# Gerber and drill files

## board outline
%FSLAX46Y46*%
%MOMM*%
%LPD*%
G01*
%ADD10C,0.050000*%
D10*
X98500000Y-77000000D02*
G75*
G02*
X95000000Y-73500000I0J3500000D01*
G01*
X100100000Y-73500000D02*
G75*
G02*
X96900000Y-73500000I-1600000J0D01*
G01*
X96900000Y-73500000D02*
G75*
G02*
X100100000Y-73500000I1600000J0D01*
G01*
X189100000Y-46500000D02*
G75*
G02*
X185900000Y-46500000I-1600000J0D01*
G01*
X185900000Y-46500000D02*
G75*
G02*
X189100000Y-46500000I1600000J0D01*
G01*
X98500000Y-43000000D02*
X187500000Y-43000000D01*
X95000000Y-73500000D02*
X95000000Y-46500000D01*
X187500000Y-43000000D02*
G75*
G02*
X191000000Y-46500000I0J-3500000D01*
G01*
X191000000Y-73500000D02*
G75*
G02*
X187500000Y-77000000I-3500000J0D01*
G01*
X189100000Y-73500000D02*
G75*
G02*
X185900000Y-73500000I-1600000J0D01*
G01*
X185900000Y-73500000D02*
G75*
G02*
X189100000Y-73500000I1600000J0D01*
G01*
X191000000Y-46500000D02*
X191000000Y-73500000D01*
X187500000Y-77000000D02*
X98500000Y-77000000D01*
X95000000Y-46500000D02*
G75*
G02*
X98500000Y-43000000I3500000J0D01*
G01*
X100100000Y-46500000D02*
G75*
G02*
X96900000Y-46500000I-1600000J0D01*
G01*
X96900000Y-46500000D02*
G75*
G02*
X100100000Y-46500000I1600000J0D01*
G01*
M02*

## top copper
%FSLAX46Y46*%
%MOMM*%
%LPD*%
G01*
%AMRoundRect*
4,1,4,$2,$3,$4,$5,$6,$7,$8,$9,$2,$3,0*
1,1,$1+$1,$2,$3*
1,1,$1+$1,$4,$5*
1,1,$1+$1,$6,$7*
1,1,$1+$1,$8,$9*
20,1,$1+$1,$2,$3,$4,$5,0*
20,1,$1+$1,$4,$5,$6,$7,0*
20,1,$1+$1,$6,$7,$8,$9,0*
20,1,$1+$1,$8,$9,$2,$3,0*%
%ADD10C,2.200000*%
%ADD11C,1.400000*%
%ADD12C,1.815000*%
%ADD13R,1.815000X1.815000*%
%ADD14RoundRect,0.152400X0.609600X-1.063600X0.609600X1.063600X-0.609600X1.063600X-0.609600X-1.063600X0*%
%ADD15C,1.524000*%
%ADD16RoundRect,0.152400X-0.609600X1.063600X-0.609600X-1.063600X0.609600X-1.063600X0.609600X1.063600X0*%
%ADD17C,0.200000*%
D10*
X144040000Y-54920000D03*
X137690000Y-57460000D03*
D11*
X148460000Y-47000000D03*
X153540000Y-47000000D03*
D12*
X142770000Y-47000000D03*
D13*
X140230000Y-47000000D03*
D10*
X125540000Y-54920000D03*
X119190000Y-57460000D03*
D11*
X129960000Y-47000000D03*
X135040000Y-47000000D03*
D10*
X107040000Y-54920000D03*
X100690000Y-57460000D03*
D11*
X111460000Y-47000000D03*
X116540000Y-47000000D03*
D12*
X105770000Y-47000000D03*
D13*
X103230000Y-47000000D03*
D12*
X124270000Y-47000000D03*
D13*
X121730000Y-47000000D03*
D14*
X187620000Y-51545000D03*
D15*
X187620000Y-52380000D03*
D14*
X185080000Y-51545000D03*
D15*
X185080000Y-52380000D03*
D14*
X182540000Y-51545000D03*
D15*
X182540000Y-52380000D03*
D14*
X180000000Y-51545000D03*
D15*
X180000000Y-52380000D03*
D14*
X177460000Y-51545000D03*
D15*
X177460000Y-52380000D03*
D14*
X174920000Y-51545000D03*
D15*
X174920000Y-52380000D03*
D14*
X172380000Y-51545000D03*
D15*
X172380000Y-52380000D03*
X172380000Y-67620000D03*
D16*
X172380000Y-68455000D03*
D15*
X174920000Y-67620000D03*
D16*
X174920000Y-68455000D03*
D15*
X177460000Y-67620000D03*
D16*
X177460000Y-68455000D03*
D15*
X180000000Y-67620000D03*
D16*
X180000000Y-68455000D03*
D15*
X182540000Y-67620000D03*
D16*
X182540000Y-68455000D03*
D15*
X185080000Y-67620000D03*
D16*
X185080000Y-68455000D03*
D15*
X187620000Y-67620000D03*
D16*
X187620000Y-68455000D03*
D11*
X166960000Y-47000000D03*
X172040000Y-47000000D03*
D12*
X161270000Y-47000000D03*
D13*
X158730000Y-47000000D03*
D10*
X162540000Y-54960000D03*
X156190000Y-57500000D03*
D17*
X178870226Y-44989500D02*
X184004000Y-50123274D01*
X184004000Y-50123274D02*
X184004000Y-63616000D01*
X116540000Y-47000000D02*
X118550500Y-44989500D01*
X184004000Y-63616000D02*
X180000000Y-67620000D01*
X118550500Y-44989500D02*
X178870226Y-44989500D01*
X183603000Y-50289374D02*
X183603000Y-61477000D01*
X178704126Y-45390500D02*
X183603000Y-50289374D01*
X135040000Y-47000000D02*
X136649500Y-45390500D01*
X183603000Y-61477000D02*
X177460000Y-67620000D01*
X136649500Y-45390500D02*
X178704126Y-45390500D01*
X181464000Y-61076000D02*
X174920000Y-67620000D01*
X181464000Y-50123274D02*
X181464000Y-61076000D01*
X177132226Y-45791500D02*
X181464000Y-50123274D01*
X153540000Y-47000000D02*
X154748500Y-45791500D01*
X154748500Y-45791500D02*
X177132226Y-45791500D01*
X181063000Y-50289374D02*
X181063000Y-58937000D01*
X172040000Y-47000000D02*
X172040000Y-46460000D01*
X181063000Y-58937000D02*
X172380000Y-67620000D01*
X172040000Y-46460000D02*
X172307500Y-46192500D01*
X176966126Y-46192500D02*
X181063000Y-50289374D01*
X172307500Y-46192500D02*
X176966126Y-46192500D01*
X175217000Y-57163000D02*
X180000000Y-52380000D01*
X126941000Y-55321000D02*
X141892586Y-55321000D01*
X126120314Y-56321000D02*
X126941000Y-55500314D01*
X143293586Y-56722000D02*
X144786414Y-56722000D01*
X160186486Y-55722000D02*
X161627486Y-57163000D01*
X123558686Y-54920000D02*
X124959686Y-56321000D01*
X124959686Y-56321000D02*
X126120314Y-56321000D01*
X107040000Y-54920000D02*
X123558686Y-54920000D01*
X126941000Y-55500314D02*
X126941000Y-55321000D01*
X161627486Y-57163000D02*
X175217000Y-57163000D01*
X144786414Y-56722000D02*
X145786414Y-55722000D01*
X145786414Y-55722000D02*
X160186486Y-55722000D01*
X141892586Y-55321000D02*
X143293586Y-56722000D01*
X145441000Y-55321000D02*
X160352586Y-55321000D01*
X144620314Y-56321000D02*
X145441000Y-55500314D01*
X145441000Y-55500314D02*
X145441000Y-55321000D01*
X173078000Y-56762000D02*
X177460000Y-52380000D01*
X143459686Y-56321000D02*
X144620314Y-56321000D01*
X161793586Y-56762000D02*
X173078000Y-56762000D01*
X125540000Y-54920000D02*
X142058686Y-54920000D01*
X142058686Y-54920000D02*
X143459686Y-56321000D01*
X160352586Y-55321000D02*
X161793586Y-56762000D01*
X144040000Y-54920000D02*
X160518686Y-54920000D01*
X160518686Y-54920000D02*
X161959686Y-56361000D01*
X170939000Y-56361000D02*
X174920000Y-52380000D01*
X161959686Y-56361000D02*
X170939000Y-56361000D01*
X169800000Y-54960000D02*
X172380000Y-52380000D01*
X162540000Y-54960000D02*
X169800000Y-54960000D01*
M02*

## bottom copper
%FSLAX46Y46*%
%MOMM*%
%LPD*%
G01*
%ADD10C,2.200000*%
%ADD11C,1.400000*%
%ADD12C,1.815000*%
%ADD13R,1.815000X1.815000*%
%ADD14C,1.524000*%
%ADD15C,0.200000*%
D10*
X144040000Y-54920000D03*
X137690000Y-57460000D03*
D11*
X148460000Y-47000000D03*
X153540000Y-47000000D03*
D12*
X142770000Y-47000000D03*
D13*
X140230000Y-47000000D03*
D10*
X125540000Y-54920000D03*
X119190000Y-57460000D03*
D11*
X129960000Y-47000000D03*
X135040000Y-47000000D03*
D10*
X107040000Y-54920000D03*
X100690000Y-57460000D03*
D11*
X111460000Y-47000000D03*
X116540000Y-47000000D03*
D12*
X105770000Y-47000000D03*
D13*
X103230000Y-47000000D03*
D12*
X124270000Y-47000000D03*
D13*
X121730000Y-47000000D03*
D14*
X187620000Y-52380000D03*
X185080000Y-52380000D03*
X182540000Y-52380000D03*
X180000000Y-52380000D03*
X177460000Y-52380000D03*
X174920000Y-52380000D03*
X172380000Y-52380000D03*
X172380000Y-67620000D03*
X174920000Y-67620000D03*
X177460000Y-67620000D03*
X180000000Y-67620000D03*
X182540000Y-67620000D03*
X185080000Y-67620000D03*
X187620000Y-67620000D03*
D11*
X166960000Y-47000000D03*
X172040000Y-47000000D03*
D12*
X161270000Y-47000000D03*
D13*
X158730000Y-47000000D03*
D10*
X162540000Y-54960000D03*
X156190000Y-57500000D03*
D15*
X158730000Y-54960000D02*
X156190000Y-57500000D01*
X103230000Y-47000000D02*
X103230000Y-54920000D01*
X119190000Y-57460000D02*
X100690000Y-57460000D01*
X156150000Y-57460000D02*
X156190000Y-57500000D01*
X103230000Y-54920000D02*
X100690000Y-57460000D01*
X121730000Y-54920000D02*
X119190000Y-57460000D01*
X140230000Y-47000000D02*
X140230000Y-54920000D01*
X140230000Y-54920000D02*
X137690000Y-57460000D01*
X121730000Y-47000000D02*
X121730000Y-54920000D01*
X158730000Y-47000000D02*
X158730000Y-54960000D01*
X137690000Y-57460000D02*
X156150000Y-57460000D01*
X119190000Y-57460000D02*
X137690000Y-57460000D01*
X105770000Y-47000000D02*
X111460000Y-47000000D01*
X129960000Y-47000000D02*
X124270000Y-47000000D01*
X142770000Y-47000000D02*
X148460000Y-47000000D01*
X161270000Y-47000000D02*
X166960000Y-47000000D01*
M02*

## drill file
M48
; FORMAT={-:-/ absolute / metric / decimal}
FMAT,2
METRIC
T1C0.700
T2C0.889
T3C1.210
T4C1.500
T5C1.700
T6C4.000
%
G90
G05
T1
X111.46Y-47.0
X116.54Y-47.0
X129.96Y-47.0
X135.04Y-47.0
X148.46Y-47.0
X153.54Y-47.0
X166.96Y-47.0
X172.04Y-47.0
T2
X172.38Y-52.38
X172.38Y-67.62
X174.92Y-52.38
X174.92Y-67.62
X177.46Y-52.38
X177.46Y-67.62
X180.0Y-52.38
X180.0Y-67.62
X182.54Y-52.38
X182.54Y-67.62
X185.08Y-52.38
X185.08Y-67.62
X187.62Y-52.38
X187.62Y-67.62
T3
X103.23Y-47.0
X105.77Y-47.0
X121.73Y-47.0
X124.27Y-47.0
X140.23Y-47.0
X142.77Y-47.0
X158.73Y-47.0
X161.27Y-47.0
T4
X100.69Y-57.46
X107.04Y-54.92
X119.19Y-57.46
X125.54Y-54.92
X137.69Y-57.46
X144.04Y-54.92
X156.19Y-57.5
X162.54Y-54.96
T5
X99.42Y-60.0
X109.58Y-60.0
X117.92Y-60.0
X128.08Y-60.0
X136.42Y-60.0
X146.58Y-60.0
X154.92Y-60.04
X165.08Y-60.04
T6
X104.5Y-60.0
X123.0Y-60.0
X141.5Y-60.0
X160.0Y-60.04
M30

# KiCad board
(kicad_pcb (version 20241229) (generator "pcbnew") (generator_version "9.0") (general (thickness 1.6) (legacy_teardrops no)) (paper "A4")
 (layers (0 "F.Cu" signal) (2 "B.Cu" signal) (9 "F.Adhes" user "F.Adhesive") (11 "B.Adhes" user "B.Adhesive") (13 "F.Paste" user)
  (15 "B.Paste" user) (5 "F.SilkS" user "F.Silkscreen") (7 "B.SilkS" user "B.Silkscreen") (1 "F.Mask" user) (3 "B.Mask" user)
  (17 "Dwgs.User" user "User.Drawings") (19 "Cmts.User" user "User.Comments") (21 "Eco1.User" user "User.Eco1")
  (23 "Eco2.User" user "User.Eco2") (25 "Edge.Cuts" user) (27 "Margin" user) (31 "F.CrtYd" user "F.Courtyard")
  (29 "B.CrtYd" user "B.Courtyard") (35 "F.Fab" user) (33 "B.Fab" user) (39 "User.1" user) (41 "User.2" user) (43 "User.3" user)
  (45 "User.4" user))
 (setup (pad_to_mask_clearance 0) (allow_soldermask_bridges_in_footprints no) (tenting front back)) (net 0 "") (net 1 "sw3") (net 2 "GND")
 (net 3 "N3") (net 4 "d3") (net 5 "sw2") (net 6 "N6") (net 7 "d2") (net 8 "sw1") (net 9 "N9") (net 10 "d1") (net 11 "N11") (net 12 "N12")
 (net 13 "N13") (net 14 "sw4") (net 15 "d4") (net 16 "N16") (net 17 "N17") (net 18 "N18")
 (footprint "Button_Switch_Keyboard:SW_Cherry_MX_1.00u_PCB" (layer "F.Cu") (at 144.04 54.92)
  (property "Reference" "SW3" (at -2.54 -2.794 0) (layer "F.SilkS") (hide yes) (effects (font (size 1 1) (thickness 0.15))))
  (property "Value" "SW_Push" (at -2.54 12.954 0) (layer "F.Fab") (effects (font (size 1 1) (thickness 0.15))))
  (pad "" np_thru_hole circle (at -7.62 5.08) (size 1.7 1.7) (drill 1.7) (layers "*.Cu" "*.Mask"))
  (pad "" np_thru_hole circle (at -2.54 5.08) (size 4 4) (drill 4) (layers "*.Cu" "*.Mask"))
  (pad "" np_thru_hole circle (at 2.54 5.08) (size 1.7 1.7) (drill 1.7) (layers "*.Cu" "*.Mask"))
  (pad "1" thru_hole circle (at 0 0) (size 2.2 2.2) (drill 1.5) (layers "*.Cu" "*.Mask") (remove_unused_layers no) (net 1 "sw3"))
  (pad "2" thru_hole circle (at -6.35 2.54) (size 2.2 2.2) (drill 1.5) (layers "*.Cu" "*.Mask") (remove_unused_layers no) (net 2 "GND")))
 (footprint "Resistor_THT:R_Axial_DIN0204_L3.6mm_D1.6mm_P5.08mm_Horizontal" (layer "F.Cu") (at 148.46 47)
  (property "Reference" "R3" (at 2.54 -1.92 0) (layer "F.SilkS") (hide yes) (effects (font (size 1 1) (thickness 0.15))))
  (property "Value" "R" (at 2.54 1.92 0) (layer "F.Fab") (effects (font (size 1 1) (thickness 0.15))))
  (pad "1" thru_hole circle (at 0 0) (size 1.4 1.4) (drill 0.7) (layers "*.Cu" "*.Mask") (remove_unused_layers no) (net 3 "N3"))
  (pad "2" thru_hole circle (at 5.08 0) (size 1.4 1.4) (drill 0.7) (layers "*.Cu" "*.Mask") (remove_unused_layers no) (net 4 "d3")))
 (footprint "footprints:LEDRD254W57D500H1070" (layer "F.Cu") (at 141.5 47)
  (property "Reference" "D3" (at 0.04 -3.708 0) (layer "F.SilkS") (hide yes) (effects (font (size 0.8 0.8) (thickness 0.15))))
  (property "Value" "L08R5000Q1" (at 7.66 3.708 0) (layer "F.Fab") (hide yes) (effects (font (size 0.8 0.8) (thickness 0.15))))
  (pad "A" thru_hole circle (at 1.27 0) (size 1.815 1.815) (drill 1.21) (layers "*.Cu" "*.Mask") (remove_unused_layers no) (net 3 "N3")
   (solder_mask_margin 0.102))
  (pad "C" thru_hole rect (at -1.27 0) (size 1.815 1.815) (drill 1.21) (layers "*.Cu" "*.Mask") (remove_unused_layers no) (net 2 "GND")
   (solder_mask_margin 0.102)))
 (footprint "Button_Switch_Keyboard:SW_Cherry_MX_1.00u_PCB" (layer "F.Cu") (at 125.54 54.92)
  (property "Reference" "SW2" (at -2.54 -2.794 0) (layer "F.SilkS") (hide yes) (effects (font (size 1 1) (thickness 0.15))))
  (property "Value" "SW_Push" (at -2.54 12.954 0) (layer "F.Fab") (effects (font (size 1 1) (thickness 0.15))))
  (pad "" np_thru_hole circle (at -7.62 5.08) (size 1.7 1.7) (drill 1.7) (layers "*.Cu" "*.Mask"))
  (pad "" np_thru_hole circle (at -2.54 5.08) (size 4 4) (drill 4) (layers "*.Cu" "*.Mask"))
  (pad "" np_thru_hole circle (at 2.54 5.08) (size 1.7 1.7) (drill 1.7) (layers "*.Cu" "*.Mask"))
  (pad "1" thru_hole circle (at 0 0) (size 2.2 2.2) (drill 1.5) (layers "*.Cu" "*.Mask") (remove_unused_layers no) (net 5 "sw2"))
  (pad "2" thru_hole circle (at -6.35 2.54) (size 2.2 2.2) (drill 1.5) (layers "*.Cu" "*.Mask") (remove_unused_layers no) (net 2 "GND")))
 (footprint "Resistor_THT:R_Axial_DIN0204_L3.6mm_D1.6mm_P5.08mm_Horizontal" (layer "F.Cu") (at 129.96 47)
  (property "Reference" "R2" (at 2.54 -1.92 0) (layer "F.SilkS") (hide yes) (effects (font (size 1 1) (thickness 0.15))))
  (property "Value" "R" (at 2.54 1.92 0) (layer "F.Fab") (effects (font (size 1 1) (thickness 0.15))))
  (pad "1" thru_hole circle (at 0 0) (size 1.4 1.4) (drill 0.7) (layers "*.Cu" "*.Mask") (remove_unused_layers no) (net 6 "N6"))
  (pad "2" thru_hole circle (at 5.08 0) (size 1.4 1.4) (drill 0.7) (layers "*.Cu" "*.Mask") (remove_unused_layers no) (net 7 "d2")))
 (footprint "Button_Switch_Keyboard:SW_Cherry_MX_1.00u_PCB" (layer "F.Cu") (at 107.04 54.92)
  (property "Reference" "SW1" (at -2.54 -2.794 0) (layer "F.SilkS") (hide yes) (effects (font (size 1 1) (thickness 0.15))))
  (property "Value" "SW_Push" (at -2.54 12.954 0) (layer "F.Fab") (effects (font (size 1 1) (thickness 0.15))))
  (pad "" np_thru_hole circle (at -7.62 5.08) (size 1.7 1.7) (drill 1.7) (layers "*.Cu" "*.Mask"))
  (pad "" np_thru_hole circle (at -2.54 5.08) (size 4 4) (drill 4) (layers "*.Cu" "*.Mask"))
  (pad "" np_thru_hole circle (at 2.54 5.08) (size 1.7 1.7) (drill 1.7) (layers "*.Cu" "*.Mask"))
  (pad "1" thru_hole circle (at 0 0) (size 2.2 2.2) (drill 1.5) (layers "*.Cu" "*.Mask") (remove_unused_layers no) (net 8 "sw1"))
  (pad "2" thru_hole circle (at -6.35 2.54) (size 2.2 2.2) (drill 1.5) (layers "*.Cu" "*.Mask") (remove_unused_layers no) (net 2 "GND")))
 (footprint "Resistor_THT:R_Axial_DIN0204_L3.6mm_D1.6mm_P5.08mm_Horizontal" (layer "F.Cu") (at 111.46 47)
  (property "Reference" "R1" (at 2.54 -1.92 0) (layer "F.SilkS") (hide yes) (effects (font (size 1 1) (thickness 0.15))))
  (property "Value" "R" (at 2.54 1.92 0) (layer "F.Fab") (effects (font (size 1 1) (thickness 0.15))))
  (pad "1" thru_hole circle (at 0 0) (size 1.4 1.4) (drill 0.7) (layers "*.Cu" "*.Mask") (remove_unused_layers no) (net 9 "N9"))
  (pad "2" thru_hole circle (at 5.08 0) (size 1.4 1.4) (drill 0.7) (layers "*.Cu" "*.Mask") (remove_unused_layers no) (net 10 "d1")))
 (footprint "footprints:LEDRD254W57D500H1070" (layer "F.Cu") (at 104.5 47)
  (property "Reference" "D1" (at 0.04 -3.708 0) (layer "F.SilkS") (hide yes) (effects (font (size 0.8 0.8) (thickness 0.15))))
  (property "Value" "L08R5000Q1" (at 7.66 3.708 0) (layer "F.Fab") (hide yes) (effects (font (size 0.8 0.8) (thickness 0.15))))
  (pad "A" thru_hole circle (at 1.27 0) (size 1.815 1.815) (drill 1.21) (layers "*.Cu" "*.Mask") (remove_unused_layers no) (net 9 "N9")
   (solder_mask_margin 0.102))
  (pad "C" thru_hole rect (at -1.27 0) (size 1.815 1.815) (drill 1.21) (layers "*.Cu" "*.Mask") (remove_unused_layers no) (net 2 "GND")
   (solder_mask_margin 0.102)))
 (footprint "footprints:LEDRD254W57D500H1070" (layer "F.Cu") (at 123 47)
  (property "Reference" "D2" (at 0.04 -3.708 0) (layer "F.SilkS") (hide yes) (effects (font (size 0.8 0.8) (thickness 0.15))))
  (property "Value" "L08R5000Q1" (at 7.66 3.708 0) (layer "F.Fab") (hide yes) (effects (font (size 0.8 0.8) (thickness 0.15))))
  (pad "A" thru_hole circle (at 1.27 0) (size 1.815 1.815) (drill 1.21) (layers "*.Cu" "*.Mask") (remove_unused_layers no) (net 6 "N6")
   (solder_mask_margin 0.102))
  (pad "C" thru_hole rect (at -1.27 0) (size 1.815 1.815) (drill 1.21) (layers "*.Cu" "*.Mask") (remove_unused_layers no) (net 2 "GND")
   (solder_mask_margin 0.102)))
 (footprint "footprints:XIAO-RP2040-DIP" (layer "F.Cu") (at 180 60 -90)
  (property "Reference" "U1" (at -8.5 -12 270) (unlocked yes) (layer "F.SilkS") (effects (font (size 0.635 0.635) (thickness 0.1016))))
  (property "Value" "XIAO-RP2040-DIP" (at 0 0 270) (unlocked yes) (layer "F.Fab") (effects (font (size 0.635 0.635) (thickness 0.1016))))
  (pad "1" smd roundrect (at -8.455 -7.62 90) (size 2.432 1.524) (layers "F.Cu" "F.Mask") (roundrect_rratio 0.1) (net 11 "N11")
   (thermal_bridge_angle 45))
  (pad "1" thru_hole circle (at -7.62 -7.62 90) (size 1.524 1.524) (drill 0.889) (layers "*.Cu" "*.Mask") (remove_unused_layers no)
   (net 11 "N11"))
  (pad "2" smd roundrect (at -8.455 -5.08 90) (size 2.432 1.524) (layers "F.Cu" "F.Mask") (roundrect_rratio 0.1) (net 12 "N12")
   (thermal_bridge_angle 45))
  (pad "2" thru_hole circle (at -7.62 -5.08 90) (size 1.524 1.524) (drill 0.889) (layers "*.Cu" "*.Mask") (remove_unused_layers no)
   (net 12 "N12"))
  (pad "3" smd roundrect (at -8.455 -2.54 90) (size 2.432 1.524) (layers "F.Cu" "F.Mask") (roundrect_rratio 0.1) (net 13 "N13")
   (thermal_bridge_angle 45))
  (pad "3" thru_hole circle (at -7.62 -2.54 90) (size 1.524 1.524) (drill 0.889) (layers "*.Cu" "*.Mask") (remove_unused_layers no)
   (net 13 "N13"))
  (pad "4" smd roundrect (at -8.455 0 90) (size 2.432 1.524) (layers "F.Cu" "F.Mask") (roundrect_rratio 0.1) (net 8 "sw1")
   (thermal_bridge_angle 45))
  (pad "4" thru_hole circle (at -7.62 0 90) (size 1.524 1.524) (drill 0.889) (layers "*.Cu" "*.Mask") (remove_unused_layers no)
   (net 8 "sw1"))
  (pad "5" smd roundrect (at -8.455 2.54 90) (size 2.432 1.524) (layers "F.Cu" "F.Mask") (roundrect_rratio 0.1) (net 5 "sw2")
   (thermal_bridge_angle 45))
  (pad "5" thru_hole circle (at -7.62 2.54 90) (size 1.524 1.524) (drill 0.889) (layers "*.Cu" "*.Mask") (remove_unused_layers no)
   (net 5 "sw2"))
  (pad "6" smd roundrect (at -8.455 5.08 90) (size 2.432 1.524) (layers "F.Cu" "F.Mask") (roundrect_rratio 0.1) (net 1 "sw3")
   (thermal_bridge_angle 45))
  (pad "6" thru_hole circle (at -7.62 5.08 90) (size 1.524 1.524) (drill 0.889) (layers "*.Cu" "*.Mask") (remove_unused_layers no)
   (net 1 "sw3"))
  (pad "7" smd roundrect (at -8.455 7.62 90) (size 2.432 1.524) (layers "F.Cu" "F.Mask") (roundrect_rratio 0.1) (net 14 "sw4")
   (thermal_bridge_angle 45))
  (pad "7" thru_hole circle (at -7.62 7.62 90) (size 1.524 1.524) (drill 0.889) (layers "*.Cu" "*.Mask") (remove_unused_layers no)
   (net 14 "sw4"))
  (pad "8" thru_hole circle (at 7.62 7.62 270) (size 1.524 1.524) (drill 0.889) (layers "*.Cu" "*.Mask") (remove_unused_layers no)
   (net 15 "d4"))
  (pad "8" smd roundrect (at 8.455 7.62 270) (size 2.432 1.524) (layers "F.Cu" "F.Mask") (roundrect_rratio 0.1) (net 15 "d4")
   (thermal_bridge_angle 45))
  (pad "9" thru_hole circle (at 7.62 5.08 270) (size 1.524 1.524) (drill 0.889) (layers "*.Cu" "*.Mask") (remove_unused_layers no)
   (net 4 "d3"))
  (pad "9" smd roundrect (at 8.455 5.08 270) (size 2.432 1.524) (layers "F.Cu" "F.Mask") (roundrect_rratio 0.1) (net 4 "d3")
   (thermal_bridge_angle 45))
  (pad "10" thru_hole circle (at 7.62 2.54 270) (size 1.524 1.524) (drill 0.889) (layers "*.Cu" "*.Mask") (remove_unused_layers no)
   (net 7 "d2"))
  (pad "10" smd roundrect (at 8.455 2.54 270) (size 2.432 1.524) (layers "F.Cu" "F.Mask") (roundrect_rratio 0.1) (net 7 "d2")
   (thermal_bridge_angle 45))
  (pad "11" thru_hole circle (at 7.62 0 270) (size 1.524 1.524) (drill 0.889) (layers "*.Cu" "*.Mask") (remove_unused_layers no)
   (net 10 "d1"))
  (pad "11" smd roundrect (at 8.455 0 270) (size 2.432 1.524) (layers "F.Cu" "F.Mask") (roundrect_rratio 0.1) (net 10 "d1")
   (thermal_bridge_angle 45))
  (pad "12" thru_hole circle (at 7.62 -2.54 270) (size 1.524 1.524) (drill 0.889) (layers "*.Cu" "*.Mask") (remove_unused_layers no)
   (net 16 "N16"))
  (pad "12" smd roundrect (at 8.455 -2.54 270) (size 2.432 1.524) (layers "F.Cu" "F.Mask") (roundrect_rratio 0.1) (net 16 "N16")
   (thermal_bridge_angle 45))
  (pad "13" thru_hole circle (at 7.62 -5.08 270) (size 1.524 1.524) (drill 0.889) (layers "*.Cu" "*.Mask") (remove_unused_layers no)
   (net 2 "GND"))
  (pad "13" smd roundrect (at 8.455 -5.08 270) (size 2.432 1.524) (layers "F.Cu" "F.Mask") (roundrect_rratio 0.1) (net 2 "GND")
   (thermal_bridge_angle 45))
  (pad "14" thru_hole circle (at 7.62 -7.62 270) (size 1.524 1.524) (drill 0.889) (layers "*.Cu" "*.Mask") (remove_unused_layers no)
   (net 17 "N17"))
  (pad "14" smd roundrect (at 8.455 -7.62 270) (size 2.432 1.524) (layers "F.Cu" "F.Mask") (roundrect_rratio 0.1) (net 17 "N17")
   (thermal_bridge_angle 45)))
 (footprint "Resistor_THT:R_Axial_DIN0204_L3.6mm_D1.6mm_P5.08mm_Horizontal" (layer "F.Cu") (at 166.96 47)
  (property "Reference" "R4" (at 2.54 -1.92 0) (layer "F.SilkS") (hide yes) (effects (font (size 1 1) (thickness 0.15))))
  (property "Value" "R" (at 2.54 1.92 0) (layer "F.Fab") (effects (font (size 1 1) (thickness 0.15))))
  (pad "1" thru_hole circle (at 0 0) (size 1.4 1.4) (drill 0.7) (layers "*.Cu" "*.Mask") (remove_unused_layers no) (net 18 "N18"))
  (pad "2" thru_hole circle (at 5.08 0) (size 1.4 1.4) (drill 0.7) (layers "*.Cu" "*.Mask") (remove_unused_layers no) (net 15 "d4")))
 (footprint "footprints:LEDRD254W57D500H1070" (layer "F.Cu") (at 160 47)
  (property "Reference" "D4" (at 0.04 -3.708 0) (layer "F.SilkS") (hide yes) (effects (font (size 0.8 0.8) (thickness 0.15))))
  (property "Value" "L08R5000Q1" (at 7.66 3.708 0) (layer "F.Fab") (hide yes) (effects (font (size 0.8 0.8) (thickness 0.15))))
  (pad "A" thru_hole circle (at 1.27 0) (size 1.815 1.815) (drill 1.21) (layers "*.Cu" "*.Mask") (remove_unused_layers no) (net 18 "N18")
   (solder_mask_margin 0.102))
  (pad "C" thru_hole rect (at -1.27 0) (size 1.815 1.815) (drill 1.21) (layers "*.Cu" "*.Mask") (remove_unused_layers no) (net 2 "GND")
   (solder_mask_margin 0.102)))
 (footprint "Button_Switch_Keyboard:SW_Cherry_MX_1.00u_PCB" (layer "F.Cu") (at 162.54 54.96)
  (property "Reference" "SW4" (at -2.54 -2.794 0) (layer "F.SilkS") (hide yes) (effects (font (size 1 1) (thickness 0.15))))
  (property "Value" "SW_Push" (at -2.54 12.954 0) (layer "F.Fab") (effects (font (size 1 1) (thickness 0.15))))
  (pad "" np_thru_hole circle (at -7.62 5.08) (size 1.7 1.7) (drill 1.7) (layers "*.Cu" "*.Mask"))
  (pad "" np_thru_hole circle (at -2.54 5.08) (size 4 4) (drill 4) (layers "*.Cu" "*.Mask"))
  (pad "" np_thru_hole circle (at 2.54 5.08) (size 1.7 1.7) (drill 1.7) (layers "*.Cu" "*.Mask"))
  (pad "1" thru_hole circle (at 0 0) (size 2.2 2.2) (drill 1.5) (layers "*.Cu" "*.Mask") (remove_unused_layers no) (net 14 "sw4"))
  (pad "2" thru_hole circle (at -6.35 2.54) (size 2.2 2.2) (drill 1.5) (layers "*.Cu" "*.Mask") (remove_unused_layers no) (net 2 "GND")))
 (gr_arc (start 98.5 77) (mid 96.025126 75.974874) (end 95 73.5) (stroke (width 0.05) (type default)) (layer "Edge.Cuts"))
 (gr_circle (center 98.5 73.5) (end 100.1 73.5) (stroke (width 0.05) (type solid)) (fill no) (layer "Edge.Cuts"))
 (gr_circle (center 187.5 46.5) (end 189.1 46.5) (stroke (width 0.05) (type solid)) (fill no) (layer "Edge.Cuts"))
 (gr_line (start 98.5 43) (end 187.5 43) (stroke (width 0.05) (type default)) (layer "Edge.Cuts"))
 (gr_line (start 95 73.5) (end 95 46.5) (stroke (width 0.05) (type default)) (layer "Edge.Cuts"))
 (gr_arc (start 187.5 43) (mid 189.974874 44.025126) (end 191 46.5) (stroke (width 0.05) (type default)) (layer "Edge.Cuts"))
 (gr_arc (start 191 73.5) (mid 189.974874 75.974874) (end 187.5 77) (stroke (width 0.05) (type default)) (layer "Edge.Cuts"))
 (gr_circle (center 187.5 73.5) (end 189.1 73.5) (stroke (width 0.05) (type solid)) (fill no) (layer "Edge.Cuts"))
 (gr_line (start 191 46.5) (end 191 73.5) (stroke (width 0.05) (type default)) (layer "Edge.Cuts"))
 (gr_line (start 187.5 77) (end 98.5 77) (stroke (width 0.05) (type default)) (layer "Edge.Cuts"))
 (gr_arc (start 95 46.5) (mid 96.025126 44.025126) (end 98.5 43) (stroke (width 0.05) (type default)) (layer "Edge.Cuts"))
 (gr_circle (center 98.5 46.5) (end 100.1 46.5) (stroke (width 0.05) (type solid)) (fill no) (layer "Edge.Cuts"))
 (segment (start 158.73 54.96) (end 156.19 57.5) (width 0.2) (layer "B.Cu") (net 2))
 (segment (start 103.23 47) (end 103.23 54.92) (width 0.2) (layer "B.Cu") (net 2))
 (segment (start 119.19 57.46) (end 100.69 57.46) (width 0.2) (layer "B.Cu") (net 2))
 (segment (start 156.15 57.46) (end 156.19 57.5) (width 0.2) (layer "B.Cu") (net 2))
 (segment (start 103.23 54.92) (end 100.69 57.46) (width 0.2) (layer "B.Cu") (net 2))
 (segment (start 121.73 54.92) (end 119.19 57.46) (width 0.2) (layer "B.Cu") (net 2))
 (segment (start 140.23 47) (end 140.23 54.92) (width 0.2) (layer "B.Cu") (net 2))
 (segment (start 140.23 54.92) (end 137.69 57.46) (width 0.2) (layer "B.Cu") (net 2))
 (segment (start 121.73 47) (end 121.73 54.92) (width 0.2) (layer "B.Cu") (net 2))
 (segment (start 158.73 47) (end 158.73 54.96) (width 0.2) (layer "B.Cu") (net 2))
 (segment (start 137.69 57.46) (end 156.15 57.46) (width 0.2) (layer "B.Cu") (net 2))
 (segment (start 119.19 57.46) (end 137.69 57.46) (width 0.2) (layer "B.Cu") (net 2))
 (segment (start 105.77 47) (end 111.46 47) (width 0.2) (layer "B.Cu") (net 9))
 (segment (start 129.96 47) (end 124.27 47) (width 0.2) (layer "B.Cu") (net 6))
 (segment (start 142.77 47) (end 148.46 47) (width 0.2) (layer "B.Cu") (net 3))
 (segment (start 161.27 47) (end 166.96 47) (width 0.2) (layer "B.Cu") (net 18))
 (segment (start 178.870226 44.9895) (end 184.004 50.123274) (width 0.2) (layer "F.Cu") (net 10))
 (segment (start 184.004 50.123274) (end 184.004 63.616) (width 0.2) (layer "F.Cu") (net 10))
 (segment (start 116.54 47) (end 118.5505 44.9895) (width 0.2) (layer "F.Cu") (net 10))
 (segment (start 184.004 63.616) (end 180 67.62) (width 0.2) (layer "F.Cu") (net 10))
 (segment (start 118.5505 44.9895) (end 178.870226 44.9895) (width 0.2) (layer "F.Cu") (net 10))
 (segment (start 183.603 50.289374) (end 183.603 61.477) (width 0.2) (layer "F.Cu") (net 7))
 (segment (start 178.704126 45.3905) (end 183.603 50.289374) (width 0.2) (layer "F.Cu") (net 7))
 (segment (start 135.04 47) (end 136.6495 45.3905) (width 0.2) (layer "F.Cu") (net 7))
 (segment (start 183.603 61.477) (end 177.46 67.62) (width 0.2) (layer "F.Cu") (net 7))
 (segment (start 136.6495 45.3905) (end 178.704126 45.3905) (width 0.2) (layer "F.Cu") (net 7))
 (segment (start 181.464 61.076) (end 174.92 67.62) (width 0.2) (layer "F.Cu") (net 4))
 (segment (start 181.464 50.123274) (end 181.464 61.076) (width 0.2) (layer "F.Cu") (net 4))
 (segment (start 177.132226 45.7915) (end 181.464 50.123274) (width 0.2) (layer "F.Cu") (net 4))
 (segment (start 153.54 47) (end 154.7485 45.7915) (width 0.2) (layer "F.Cu") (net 4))
 (segment (start 154.7485 45.7915) (end 177.132226 45.7915) (width 0.2) (layer "F.Cu") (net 4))
 (segment (start 181.063 50.289374) (end 181.063 58.937) (width 0.2) (layer "F.Cu") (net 15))
 (segment (start 172.04 47) (end 172.04 46.46) (width 0.2) (layer "F.Cu") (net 15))
 (segment (start 181.063 58.937) (end 172.38 67.62) (width 0.2) (layer "F.Cu") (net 15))
 (segment (start 172.04 46.46) (end 172.3075 46.1925) (width 0.2) (layer "F.Cu") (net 15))
 (segment (start 176.966126 46.1925) (end 181.063 50.289374) (width 0.2) (layer "F.Cu") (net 15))
 (segment (start 172.3075 46.1925) (end 176.966126 46.1925) (width 0.2) (layer "F.Cu") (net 15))
 (segment (start 175.217 57.163) (end 180 52.38) (width 0.2) (layer "F.Cu") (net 8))
 (segment (start 126.941 55.321) (end 141.892586 55.321) (width 0.2) (layer "F.Cu") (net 8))
 (segment (start 126.120314 56.321) (end 126.941 55.500314) (width 0.2) (layer "F.Cu") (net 8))
 (segment (start 143.293586 56.722) (end 144.786414 56.722) (width 0.2) (layer "F.Cu") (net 8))
 (segment (start 160.186486 55.722) (end 161.627486 57.163) (width 0.2) (layer "F.Cu") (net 8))
 (segment (start 123.558686 54.92) (end 124.959686 56.321) (width 0.2) (layer "F.Cu") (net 8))
 (segment (start 124.959686 56.321) (end 126.120314 56.321) (width 0.2) (layer "F.Cu") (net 8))
 (segment (start 107.04 54.92) (end 123.558686 54.92) (width 0.2) (layer "F.Cu") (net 8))
 (segment (start 126.941 55.500314) (end 126.941 55.321) (width 0.2) (layer "F.Cu") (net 8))
 (segment (start 161.627486 57.163) (end 175.217 57.163) (width 0.2) (layer "F.Cu") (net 8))
 (segment (start 144.786414 56.722) (end 145.786414 55.722) (width 0.2) (layer "F.Cu") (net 8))
 (segment (start 145.786414 55.722) (end 160.186486 55.722) (width 0.2) (layer "F.Cu") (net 8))
 (segment (start 141.892586 55.321) (end 143.293586 56.722) (width 0.2) (layer "F.Cu") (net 8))
 (segment (start 145.441 55.321) (end 160.352586 55.321) (width 0.2) (layer "F.Cu") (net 5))
 (segment (start 144.620314 56.321) (end 145.441 55.500314) (width 0.2) (layer "F.Cu") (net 5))
 (segment (start 145.441 55.500314) (end 145.441 55.321) (width 0.2) (layer "F.Cu") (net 5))
 (segment (start 173.078 56.762) (end 177.46 52.38) (width 0.2) (layer "F.Cu") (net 5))
 (segment (start 143.459686 56.321) (end 144.620314 56.321) (width 0.2) (layer "F.Cu") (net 5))
 (segment (start 161.793586 56.762) (end 173.078 56.762) (width 0.2) (layer "F.Cu") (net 5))
 (segment (start 125.54 54.92) (end 142.058686 54.92) (width 0.2) (layer "F.Cu") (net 5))
 (segment (start 142.058686 54.92) (end 143.459686 56.321) (width 0.2) (layer "F.Cu") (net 5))
 (segment (start 160.352586 55.321) (end 161.793586 56.762) (width 0.2) (layer "F.Cu") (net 5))
 (segment (start 144.04 54.92) (end 160.518686 54.92) (width 0.2) (layer "F.Cu") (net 1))
 (segment (start 160.518686 54.92) (end 161.959686 56.361) (width 0.2) (layer "F.Cu") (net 1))
 (segment (start 170.939 56.361) (end 174.92 52.38) (width 0.2) (layer "F.Cu") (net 1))
 (segment (start 161.959686 56.361) (end 170.939 56.361) (width 0.2) (layer "F.Cu") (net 1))
 (segment (start 169.8 54.96) (end 172.38 52.38) (width 0.2) (layer "F.Cu") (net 14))
 (segment (start 162.54 54.96) (end 169.8 54.96) (width 0.2) (layer "F.Cu") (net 14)))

